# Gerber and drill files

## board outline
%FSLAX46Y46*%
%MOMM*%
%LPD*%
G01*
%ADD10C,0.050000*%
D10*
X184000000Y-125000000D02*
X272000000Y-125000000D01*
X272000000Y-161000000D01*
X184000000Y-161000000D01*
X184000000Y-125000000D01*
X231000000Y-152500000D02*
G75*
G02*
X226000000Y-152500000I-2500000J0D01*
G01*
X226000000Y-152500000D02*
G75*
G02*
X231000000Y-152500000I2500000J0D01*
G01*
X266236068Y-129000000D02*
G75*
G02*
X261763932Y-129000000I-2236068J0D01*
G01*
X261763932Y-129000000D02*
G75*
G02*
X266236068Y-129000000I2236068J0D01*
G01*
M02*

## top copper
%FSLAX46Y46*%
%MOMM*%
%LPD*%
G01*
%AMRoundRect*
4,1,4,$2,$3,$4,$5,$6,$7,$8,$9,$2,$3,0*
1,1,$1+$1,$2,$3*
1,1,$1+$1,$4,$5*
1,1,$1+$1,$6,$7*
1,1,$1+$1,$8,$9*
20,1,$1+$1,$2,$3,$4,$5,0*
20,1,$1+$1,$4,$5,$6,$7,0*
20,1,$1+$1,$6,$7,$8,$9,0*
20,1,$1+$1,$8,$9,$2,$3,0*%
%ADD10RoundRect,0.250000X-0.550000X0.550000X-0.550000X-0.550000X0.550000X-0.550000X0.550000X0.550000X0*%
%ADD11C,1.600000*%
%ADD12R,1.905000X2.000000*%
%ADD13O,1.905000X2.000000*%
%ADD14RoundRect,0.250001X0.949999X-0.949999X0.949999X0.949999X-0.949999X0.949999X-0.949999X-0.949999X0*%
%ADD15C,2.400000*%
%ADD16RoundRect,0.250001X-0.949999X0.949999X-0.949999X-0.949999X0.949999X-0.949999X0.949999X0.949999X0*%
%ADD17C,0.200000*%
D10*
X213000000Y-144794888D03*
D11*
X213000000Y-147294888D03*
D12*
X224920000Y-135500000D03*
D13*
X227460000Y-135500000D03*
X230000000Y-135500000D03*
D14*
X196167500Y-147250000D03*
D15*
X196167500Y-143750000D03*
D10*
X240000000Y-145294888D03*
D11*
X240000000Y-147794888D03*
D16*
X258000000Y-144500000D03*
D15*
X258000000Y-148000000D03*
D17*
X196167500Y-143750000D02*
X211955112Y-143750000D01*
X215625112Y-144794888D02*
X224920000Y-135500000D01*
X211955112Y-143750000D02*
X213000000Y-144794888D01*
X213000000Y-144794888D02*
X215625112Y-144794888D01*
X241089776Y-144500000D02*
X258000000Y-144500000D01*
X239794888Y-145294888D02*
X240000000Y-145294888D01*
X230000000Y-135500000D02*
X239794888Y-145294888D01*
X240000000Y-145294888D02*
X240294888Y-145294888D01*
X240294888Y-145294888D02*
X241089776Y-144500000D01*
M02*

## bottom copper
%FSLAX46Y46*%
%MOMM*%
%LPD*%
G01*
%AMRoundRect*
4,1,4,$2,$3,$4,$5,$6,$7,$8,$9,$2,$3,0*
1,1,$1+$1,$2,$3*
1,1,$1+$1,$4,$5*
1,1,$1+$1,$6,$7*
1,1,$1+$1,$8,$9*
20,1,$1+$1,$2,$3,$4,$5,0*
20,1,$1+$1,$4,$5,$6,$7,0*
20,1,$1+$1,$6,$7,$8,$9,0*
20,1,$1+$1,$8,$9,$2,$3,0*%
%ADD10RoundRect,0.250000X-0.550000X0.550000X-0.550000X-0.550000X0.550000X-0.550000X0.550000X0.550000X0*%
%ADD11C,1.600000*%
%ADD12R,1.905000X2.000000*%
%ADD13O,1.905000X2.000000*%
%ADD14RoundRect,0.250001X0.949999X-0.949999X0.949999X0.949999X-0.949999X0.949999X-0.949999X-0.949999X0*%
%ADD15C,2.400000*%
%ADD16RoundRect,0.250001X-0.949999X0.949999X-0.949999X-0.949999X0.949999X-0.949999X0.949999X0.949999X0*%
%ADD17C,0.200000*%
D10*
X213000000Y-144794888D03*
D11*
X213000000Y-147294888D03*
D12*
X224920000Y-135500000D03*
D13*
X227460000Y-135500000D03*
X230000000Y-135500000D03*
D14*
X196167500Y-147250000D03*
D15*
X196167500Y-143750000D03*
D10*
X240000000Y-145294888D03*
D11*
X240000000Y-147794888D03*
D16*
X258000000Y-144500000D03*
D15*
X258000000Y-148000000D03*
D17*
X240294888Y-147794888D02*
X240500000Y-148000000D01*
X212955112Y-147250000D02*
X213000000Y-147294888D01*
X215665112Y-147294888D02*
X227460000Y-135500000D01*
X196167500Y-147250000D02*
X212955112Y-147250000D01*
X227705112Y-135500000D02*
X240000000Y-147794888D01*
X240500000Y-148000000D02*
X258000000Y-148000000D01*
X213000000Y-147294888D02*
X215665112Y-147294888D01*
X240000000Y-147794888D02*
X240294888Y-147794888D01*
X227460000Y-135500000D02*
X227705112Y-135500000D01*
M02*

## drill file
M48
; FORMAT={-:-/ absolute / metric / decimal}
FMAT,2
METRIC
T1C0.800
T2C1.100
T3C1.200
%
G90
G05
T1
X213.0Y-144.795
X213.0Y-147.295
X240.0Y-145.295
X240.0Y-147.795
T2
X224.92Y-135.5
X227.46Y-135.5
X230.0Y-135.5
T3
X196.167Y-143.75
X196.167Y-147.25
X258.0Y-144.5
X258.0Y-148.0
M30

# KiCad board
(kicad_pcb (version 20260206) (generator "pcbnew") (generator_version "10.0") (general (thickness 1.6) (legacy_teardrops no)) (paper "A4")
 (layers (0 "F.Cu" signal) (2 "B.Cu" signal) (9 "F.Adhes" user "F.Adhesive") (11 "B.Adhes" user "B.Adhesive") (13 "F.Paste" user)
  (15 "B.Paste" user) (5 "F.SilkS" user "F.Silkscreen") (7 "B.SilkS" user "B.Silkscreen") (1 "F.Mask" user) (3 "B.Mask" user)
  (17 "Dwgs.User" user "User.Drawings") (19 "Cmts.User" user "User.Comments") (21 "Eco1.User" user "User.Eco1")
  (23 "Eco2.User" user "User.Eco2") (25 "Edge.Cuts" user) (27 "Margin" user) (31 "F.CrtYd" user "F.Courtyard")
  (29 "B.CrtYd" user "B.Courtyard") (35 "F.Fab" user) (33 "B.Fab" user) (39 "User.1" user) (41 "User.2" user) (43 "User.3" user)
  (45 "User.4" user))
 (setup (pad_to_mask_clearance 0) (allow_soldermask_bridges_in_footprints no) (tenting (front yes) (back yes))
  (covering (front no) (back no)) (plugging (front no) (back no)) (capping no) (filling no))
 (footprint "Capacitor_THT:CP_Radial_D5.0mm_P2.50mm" (layer "F.Cu") (at 213 144.794888 -90)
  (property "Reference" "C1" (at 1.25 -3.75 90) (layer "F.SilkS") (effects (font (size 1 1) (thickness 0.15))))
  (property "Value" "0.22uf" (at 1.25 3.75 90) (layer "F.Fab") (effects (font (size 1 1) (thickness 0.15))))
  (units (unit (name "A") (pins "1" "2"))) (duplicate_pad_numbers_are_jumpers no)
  (pad "1" thru_hole roundrect (at 0 0 270) (size 1.6 1.6) (drill 0.8) (layers "*.Cu" "*.Mask") (remove_unused_layers no)
   (roundrect_rratio 0.15625) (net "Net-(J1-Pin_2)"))
  (pad "2" thru_hole circle (at 2.5 0 270) (size 1.6 1.6) (drill 0.8) (layers "*.Cu" "*.Mask") (remove_unused_layers no) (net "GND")))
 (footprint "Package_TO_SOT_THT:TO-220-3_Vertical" (layer "F.Cu") (at 224.92 135.5)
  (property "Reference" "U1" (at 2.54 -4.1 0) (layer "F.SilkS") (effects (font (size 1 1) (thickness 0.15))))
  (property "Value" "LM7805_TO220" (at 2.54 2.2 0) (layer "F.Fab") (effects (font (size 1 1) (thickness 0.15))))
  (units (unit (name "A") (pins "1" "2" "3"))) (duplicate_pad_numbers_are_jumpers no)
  (pad "1" thru_hole rect (at 0 0) (size 1.905 2) (drill 1.1) (layers "*.Cu" "*.Mask") (remove_unused_layers no) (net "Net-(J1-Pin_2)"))
  (pad "2" thru_hole oval (at 2.54 0) (size 1.905 2) (drill 1.1) (layers "*.Cu" "*.Mask") (remove_unused_layers no) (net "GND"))
  (pad "3" thru_hole oval (at 5.08 0) (size 1.905 2) (drill 1.1) (layers "*.Cu" "*.Mask") (remove_unused_layers no) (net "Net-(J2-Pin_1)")))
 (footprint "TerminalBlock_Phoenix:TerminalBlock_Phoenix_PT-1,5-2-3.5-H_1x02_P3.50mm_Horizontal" (layer "F.Cu") (at 196.1675 147.25 90)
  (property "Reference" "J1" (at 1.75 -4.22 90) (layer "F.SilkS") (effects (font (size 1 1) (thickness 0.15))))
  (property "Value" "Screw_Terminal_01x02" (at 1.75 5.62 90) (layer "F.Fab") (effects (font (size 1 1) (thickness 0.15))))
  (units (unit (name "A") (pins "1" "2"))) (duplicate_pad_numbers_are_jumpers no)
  (pad "1" thru_hole roundrect (at 0 0 90) (size 2.4 2.4) (drill 1.2) (layers "*.Cu" "*.Mask") (remove_unused_layers no)
   (roundrect_rratio 0.104167) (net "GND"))
  (pad "2" thru_hole circle (at 3.5 0 90) (size 2.4 2.4) (drill 1.2) (layers "*.Cu" "*.Mask") (remove_unused_layers no)
   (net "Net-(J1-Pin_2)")))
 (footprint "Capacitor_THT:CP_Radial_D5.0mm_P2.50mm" (layer "F.Cu") (at 240 145.294888 -90)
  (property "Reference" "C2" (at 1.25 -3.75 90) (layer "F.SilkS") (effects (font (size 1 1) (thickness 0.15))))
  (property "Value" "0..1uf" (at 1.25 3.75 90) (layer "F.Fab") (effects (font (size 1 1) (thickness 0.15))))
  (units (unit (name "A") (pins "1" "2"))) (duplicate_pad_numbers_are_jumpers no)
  (pad "1" thru_hole roundrect (at 0 0 270) (size 1.6 1.6) (drill 0.8) (layers "*.Cu" "*.Mask") (remove_unused_layers no)
   (roundrect_rratio 0.15625) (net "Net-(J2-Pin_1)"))
  (pad "2" thru_hole circle (at 2.5 0 270) (size 1.6 1.6) (drill 0.8) (layers "*.Cu" "*.Mask") (remove_unused_layers no) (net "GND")))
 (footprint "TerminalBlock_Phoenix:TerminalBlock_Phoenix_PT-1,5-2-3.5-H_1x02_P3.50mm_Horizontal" (layer "F.Cu") (at 258 144.5 -90)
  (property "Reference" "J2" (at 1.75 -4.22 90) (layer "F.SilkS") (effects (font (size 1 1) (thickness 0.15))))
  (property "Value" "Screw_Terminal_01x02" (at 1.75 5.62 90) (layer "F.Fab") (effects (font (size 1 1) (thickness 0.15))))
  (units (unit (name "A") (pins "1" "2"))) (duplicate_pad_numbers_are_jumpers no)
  (pad "1" thru_hole roundrect (at 0 0 270) (size 2.4 2.4) (drill 1.2) (layers "*.Cu" "*.Mask") (remove_unused_layers no)
   (roundrect_rratio 0.104167) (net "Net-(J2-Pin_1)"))
  (pad "2" thru_hole circle (at 3.5 0 270) (size 2.4 2.4) (drill 1.2) (layers "*.Cu" "*.Mask") (remove_unused_layers no) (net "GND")))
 (gr_rect (start 184 125) (end 272 161) (stroke (width 0.05) (type default)) (fill no) (layer "Edge.Cuts"))
 (gr_circle (center 228.5 152.5) (end 227 154.5) (stroke (width 0.05) (type default)) (fill no) (layer "Edge.Cuts"))
 (gr_circle (center 264 129) (end 263 131) (stroke (width 0.05) (type default)) (fill no) (layer "Edge.Cuts"))
 (segment (start 196.1675 143.75) (end 211.955112 143.75) (width 0.2) (layer "F.Cu") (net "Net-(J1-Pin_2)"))
 (segment (start 215.625112 144.794888) (end 224.92 135.5) (width 0.2) (layer "F.Cu") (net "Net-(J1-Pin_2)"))
 (segment (start 211.955112 143.75) (end 213 144.794888) (width 0.2) (layer "F.Cu") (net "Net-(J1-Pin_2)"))
 (segment (start 213 144.794888) (end 215.625112 144.794888) (width 0.2) (layer "F.Cu") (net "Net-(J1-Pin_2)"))
 (segment (start 240.294888 147.794888) (end 240.5 148) (width 0.2) (layer "B.Cu") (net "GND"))
 (segment (start 212.955112 147.25) (end 213 147.294888) (width 0.2) (layer "B.Cu") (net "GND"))
 (segment (start 215.665112 147.294888) (end 227.46 135.5) (width 0.2) (layer "B.Cu") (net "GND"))
 (segment (start 196.1675 147.25) (end 212.955112 147.25) (width 0.2) (layer "B.Cu") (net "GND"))
 (segment (start 227.705112 135.5) (end 240 147.794888) (width 0.2) (layer "B.Cu") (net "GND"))
 (segment (start 240.5 148) (end 258 148) (width 0.2) (layer "B.Cu") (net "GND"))
 (segment (start 213 147.294888) (end 215.665112 147.294888) (width 0.2) (layer "B.Cu") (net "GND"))
 (segment (start 240 147.794888) (end 240.294888 147.794888) (width 0.2) (layer "B.Cu") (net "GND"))
 (segment (start 227.46 135.5) (end 227.705112 135.5) (width 0.2) (layer "B.Cu") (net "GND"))
 (segment (start 241.089776 144.5) (end 258 144.5) (width 0.2) (layer "F.Cu") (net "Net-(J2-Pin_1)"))
 (segment (start 239.794888 145.294888) (end 240 145.294888) (width 0.2) (layer "F.Cu") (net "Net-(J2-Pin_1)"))
 (segment (start 230 135.5) (end 239.794888 145.294888) (width 0.2) (layer "F.Cu") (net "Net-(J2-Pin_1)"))
 (segment (start 240 145.294888) (end 240.294888 145.294888) (width 0.2) (layer "F.Cu") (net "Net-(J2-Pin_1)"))
 (segment (start 240.294888 145.294888) (end 241.089776 144.5) (width 0.2) (layer "F.Cu") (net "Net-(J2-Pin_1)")))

